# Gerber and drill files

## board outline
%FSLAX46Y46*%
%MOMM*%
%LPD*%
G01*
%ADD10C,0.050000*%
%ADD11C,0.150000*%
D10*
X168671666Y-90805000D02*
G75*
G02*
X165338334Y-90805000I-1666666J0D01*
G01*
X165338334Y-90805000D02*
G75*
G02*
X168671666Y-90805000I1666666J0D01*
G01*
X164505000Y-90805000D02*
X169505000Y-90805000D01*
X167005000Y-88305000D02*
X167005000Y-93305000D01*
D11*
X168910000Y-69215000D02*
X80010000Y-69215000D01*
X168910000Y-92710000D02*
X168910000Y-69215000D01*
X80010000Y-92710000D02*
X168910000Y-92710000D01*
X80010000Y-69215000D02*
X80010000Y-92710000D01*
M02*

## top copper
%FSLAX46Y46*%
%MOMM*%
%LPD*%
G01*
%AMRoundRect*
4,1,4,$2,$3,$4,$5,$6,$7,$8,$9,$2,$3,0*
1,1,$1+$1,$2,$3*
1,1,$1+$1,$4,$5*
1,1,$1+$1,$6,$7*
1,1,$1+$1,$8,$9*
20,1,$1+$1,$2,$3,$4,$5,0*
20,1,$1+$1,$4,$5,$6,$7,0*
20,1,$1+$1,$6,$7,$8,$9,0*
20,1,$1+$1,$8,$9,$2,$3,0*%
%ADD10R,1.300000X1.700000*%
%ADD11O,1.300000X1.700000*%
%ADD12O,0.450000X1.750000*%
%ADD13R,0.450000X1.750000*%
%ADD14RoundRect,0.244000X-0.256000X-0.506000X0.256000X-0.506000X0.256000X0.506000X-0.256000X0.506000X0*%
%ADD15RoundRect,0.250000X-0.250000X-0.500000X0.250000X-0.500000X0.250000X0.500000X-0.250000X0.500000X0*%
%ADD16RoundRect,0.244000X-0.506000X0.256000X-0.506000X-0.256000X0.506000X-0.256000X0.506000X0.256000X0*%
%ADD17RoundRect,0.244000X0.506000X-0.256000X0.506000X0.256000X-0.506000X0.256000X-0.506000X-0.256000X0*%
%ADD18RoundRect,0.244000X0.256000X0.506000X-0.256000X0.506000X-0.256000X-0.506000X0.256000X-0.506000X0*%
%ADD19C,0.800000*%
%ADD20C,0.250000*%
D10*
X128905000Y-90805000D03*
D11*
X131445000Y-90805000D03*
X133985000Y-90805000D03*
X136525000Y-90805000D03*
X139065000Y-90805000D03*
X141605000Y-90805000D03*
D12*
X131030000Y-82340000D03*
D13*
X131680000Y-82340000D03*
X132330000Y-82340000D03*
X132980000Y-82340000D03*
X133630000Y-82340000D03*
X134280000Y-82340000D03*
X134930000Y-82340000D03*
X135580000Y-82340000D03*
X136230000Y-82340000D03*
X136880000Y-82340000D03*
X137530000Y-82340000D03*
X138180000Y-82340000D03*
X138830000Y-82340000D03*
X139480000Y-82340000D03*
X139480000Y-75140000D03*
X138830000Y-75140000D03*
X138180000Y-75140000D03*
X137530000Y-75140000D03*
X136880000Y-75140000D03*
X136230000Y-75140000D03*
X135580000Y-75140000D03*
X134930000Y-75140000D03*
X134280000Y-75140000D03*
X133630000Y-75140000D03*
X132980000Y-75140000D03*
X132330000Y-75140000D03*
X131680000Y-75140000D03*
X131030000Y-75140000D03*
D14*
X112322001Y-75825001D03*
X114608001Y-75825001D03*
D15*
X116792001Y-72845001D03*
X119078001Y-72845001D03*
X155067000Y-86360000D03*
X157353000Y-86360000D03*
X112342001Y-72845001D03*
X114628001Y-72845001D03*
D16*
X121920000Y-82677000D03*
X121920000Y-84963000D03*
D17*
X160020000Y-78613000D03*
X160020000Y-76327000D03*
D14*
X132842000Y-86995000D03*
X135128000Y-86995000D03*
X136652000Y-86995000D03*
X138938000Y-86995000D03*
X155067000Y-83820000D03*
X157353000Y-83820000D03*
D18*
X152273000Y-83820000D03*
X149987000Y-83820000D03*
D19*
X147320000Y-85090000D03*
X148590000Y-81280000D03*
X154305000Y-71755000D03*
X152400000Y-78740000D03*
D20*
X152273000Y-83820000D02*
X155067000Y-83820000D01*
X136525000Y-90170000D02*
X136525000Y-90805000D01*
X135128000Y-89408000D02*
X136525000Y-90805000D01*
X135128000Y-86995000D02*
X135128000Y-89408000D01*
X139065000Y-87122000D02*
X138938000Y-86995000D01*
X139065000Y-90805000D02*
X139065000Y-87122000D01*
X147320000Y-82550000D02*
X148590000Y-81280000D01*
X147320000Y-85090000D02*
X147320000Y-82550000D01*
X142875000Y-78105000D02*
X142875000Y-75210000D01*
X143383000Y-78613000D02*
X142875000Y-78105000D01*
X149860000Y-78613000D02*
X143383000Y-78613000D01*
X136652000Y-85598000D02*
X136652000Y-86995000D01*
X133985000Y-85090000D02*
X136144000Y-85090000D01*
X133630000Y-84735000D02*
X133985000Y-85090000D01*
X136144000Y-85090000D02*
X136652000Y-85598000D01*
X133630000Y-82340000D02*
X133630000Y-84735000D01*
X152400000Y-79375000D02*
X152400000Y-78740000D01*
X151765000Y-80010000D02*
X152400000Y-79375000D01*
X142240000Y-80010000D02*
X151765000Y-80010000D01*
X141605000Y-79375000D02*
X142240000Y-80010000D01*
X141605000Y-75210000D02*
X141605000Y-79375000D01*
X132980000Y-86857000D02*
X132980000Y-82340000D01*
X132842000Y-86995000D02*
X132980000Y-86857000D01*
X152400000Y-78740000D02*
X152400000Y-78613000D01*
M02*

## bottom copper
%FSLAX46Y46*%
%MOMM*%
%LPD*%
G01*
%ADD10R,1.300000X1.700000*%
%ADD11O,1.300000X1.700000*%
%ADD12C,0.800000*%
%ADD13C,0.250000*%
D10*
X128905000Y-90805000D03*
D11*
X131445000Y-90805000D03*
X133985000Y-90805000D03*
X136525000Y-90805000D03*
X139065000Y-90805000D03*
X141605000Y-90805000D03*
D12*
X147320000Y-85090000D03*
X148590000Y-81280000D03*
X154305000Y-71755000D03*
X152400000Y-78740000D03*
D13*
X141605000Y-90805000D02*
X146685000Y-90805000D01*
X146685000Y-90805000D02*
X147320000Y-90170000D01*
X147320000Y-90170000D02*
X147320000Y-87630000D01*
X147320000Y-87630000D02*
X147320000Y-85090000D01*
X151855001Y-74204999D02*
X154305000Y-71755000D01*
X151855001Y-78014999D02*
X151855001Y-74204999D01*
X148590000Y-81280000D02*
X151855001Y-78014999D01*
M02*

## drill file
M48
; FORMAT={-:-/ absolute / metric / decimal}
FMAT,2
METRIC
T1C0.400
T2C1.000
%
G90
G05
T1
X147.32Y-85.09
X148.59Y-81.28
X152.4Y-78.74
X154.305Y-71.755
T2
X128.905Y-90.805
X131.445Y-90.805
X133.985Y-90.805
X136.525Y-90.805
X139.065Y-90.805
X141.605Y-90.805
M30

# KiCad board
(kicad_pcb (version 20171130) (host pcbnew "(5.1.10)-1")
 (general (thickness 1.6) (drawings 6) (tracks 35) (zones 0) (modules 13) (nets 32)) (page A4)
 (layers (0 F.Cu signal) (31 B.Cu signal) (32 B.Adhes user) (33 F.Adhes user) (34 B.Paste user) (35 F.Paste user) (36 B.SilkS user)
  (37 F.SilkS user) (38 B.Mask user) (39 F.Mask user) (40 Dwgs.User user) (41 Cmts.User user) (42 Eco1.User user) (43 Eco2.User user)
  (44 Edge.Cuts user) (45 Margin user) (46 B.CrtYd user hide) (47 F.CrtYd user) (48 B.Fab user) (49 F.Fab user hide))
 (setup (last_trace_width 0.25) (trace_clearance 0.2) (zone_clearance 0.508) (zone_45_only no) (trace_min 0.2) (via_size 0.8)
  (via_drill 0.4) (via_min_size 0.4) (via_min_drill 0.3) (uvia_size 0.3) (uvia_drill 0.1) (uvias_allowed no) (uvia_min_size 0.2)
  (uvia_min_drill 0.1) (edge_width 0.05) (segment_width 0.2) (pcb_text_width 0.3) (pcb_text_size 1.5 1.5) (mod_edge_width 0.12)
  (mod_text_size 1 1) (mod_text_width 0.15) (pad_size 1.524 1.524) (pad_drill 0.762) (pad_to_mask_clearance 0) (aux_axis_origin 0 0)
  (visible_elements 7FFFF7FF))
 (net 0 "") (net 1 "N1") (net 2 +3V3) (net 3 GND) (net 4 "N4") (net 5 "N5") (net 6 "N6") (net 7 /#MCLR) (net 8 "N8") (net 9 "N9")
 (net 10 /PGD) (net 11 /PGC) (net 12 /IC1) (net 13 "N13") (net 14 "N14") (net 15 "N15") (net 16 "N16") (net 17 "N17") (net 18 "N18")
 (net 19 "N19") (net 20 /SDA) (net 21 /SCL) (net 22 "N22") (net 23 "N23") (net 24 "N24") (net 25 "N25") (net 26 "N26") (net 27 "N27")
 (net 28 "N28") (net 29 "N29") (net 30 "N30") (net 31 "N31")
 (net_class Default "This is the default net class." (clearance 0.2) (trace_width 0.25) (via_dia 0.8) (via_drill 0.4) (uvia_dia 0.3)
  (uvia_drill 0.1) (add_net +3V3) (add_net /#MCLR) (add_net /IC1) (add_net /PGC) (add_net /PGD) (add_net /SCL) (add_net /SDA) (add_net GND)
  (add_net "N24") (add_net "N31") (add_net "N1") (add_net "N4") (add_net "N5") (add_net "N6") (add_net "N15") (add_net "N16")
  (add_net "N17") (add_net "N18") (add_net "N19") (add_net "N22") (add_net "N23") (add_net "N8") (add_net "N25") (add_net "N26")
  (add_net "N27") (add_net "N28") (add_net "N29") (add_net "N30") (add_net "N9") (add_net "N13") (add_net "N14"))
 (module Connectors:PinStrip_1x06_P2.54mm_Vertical (layer F.Cu) (at 128.905 90.805 90)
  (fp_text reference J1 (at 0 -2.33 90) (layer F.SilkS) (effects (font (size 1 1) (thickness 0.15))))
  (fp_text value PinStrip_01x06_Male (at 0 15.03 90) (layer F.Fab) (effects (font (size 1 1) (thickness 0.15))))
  (pad 1 thru_hole rect (at 0 0 90) (size 1.7 1.3) (drill 1) (layers *.Cu *.Mask) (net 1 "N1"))
  (pad 2 thru_hole oval (at 0 2.54 90) (size 1.7 1.3) (drill 1) (layers *.Cu *.Mask) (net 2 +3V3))
  (pad 3 thru_hole oval (at 0 5.08 90) (size 1.7 1.3) (drill 1) (layers *.Cu *.Mask) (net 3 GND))
  (pad 4 thru_hole oval (at 0 7.62 90) (size 1.7 1.3) (drill 1) (layers *.Cu *.Mask) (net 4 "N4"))
  (pad 5 thru_hole oval (at 0 10.16 90) (size 1.7 1.3) (drill 1) (layers *.Cu *.Mask) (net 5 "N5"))
  (pad 6 thru_hole oval (at 0 12.7 90) (size 1.7 1.3) (drill 1) (layers *.Cu *.Mask) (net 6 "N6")))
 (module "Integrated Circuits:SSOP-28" (layer F.Cu) (at 135.255 78.74 90)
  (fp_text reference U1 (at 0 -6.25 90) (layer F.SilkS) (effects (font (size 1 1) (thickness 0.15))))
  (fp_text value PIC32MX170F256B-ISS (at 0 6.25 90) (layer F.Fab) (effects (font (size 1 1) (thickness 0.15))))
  (pad 1 smd oval (at -3.6 -4.225 90) (size 1.75 0.45) (layers F.Cu F.Paste F.Mask) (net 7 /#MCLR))
  (pad 2 smd rect (at -3.6 -3.575 90) (size 1.75 0.45) (layers F.Cu F.Paste F.Mask) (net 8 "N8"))
  (pad 3 smd rect (at -3.6 -2.925 90) (size 1.75 0.45) (layers F.Cu F.Paste F.Mask) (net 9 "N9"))
  (pad 4 smd rect (at -3.6 -2.275 90) (size 1.75 0.45) (layers F.Cu F.Paste F.Mask) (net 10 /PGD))
  (pad 5 smd rect (at -3.6 -1.625 90) (size 1.75 0.45) (layers F.Cu F.Paste F.Mask) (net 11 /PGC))
  (pad 6 smd rect (at -3.6 -0.975 90) (size 1.75 0.45) (layers F.Cu F.Paste F.Mask) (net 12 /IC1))
  (pad 7 smd rect (at -3.6 -0.325 90) (size 1.75 0.45) (layers F.Cu F.Paste F.Mask) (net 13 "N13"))
  (pad 8 smd rect (at -3.6 0.325 90) (size 1.75 0.45) (layers F.Cu F.Paste F.Mask) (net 3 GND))
  (pad 9 smd rect (at -3.6 0.975 90) (size 1.75 0.45) (layers F.Cu F.Paste F.Mask) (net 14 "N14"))
  (pad 10 smd rect (at -3.6 1.625 90) (size 1.75 0.45) (layers F.Cu F.Paste F.Mask) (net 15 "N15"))
  (pad 11 smd rect (at -3.6 2.275 90) (size 1.75 0.45) (layers F.Cu F.Paste F.Mask) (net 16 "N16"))
  (pad 12 smd rect (at -3.6 2.925 90) (size 1.75 0.45) (layers F.Cu F.Paste F.Mask) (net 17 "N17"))
  (pad 13 smd rect (at -3.6 3.575 90) (size 1.75 0.45) (layers F.Cu F.Paste F.Mask) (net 2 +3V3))
  (pad 14 smd rect (at -3.6 4.225 90) (size 1.75 0.45) (layers F.Cu F.Paste F.Mask) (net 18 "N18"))
  (pad 15 smd rect (at 3.6 4.225 90) (size 1.75 0.45) (layers F.Cu F.Paste F.Mask) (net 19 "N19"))
  (pad 16 smd rect (at 3.6 3.575 90) (size 1.75 0.45) (layers F.Cu F.Paste F.Mask) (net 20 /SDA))
  (pad 17 smd rect (at 3.6 2.925 90) (size 1.75 0.45) (layers F.Cu F.Paste F.Mask) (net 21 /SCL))
  (pad 18 smd rect (at 3.6 2.275 90) (size 1.75 0.45) (layers F.Cu F.Paste F.Mask) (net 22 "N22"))
  (pad 19 smd rect (at 3.6 1.625 90) (size 1.75 0.45) (layers F.Cu F.Paste F.Mask) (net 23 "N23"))
  (pad 20 smd rect (at 3.6 0.975 90) (size 1.75 0.45) (layers F.Cu F.Paste F.Mask) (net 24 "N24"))
  (pad 21 smd rect (at 3.6 0.325 90) (size 1.75 0.45) (layers F.Cu F.Paste F.Mask) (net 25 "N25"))
  (pad 22 smd rect (at 3.6 -0.325 90) (size 1.75 0.45) (layers F.Cu F.Paste F.Mask) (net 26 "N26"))
  (pad 23 smd rect (at 3.6 -0.975 90) (size 1.75 0.45) (layers F.Cu F.Paste F.Mask) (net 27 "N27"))
  (pad 24 smd rect (at 3.6 -1.625 90) (size 1.75 0.45) (layers F.Cu F.Paste F.Mask) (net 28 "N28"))
  (pad 25 smd rect (at 3.6 -2.275 90) (size 1.75 0.45) (layers F.Cu F.Paste F.Mask) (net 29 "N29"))
  (pad 26 smd rect (at 3.6 -2.925 90) (size 1.75 0.45) (layers F.Cu F.Paste F.Mask) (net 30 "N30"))
  (pad 27 smd rect (at 3.6 -3.575 90) (size 1.75 0.45) (layers F.Cu F.Paste F.Mask) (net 3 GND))
  (pad 28 smd rect (at 3.6 -4.225 90) (size 1.75 0.45) (layers F.Cu F.Paste F.Mask) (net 2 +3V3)))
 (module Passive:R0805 (layer F.Cu) (at 113.465001 75.825001)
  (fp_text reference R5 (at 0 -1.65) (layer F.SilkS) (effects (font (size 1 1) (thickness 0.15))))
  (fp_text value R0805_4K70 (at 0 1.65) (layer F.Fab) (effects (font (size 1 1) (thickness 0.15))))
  (pad 1 smd roundrect (at -1.143 0) (size 1 1.5) (layers F.Cu F.Paste F.Mask) (roundrect_rratio 0.244) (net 2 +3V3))
  (pad 2 smd roundrect (at 1.143 0) (size 1 1.5) (layers F.Cu F.Paste F.Mask) (roundrect_rratio 0.244) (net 7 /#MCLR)))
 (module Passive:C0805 (layer F.Cu) (at 117.935001 72.845001)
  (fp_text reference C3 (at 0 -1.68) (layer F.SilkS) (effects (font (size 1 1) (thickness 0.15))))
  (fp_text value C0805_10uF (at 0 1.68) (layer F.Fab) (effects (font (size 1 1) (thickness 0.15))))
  (pad 1 smd roundrect (at -1.143 0) (size 1 1.5) (layers F.Cu F.Paste F.Mask) (roundrect_rratio 0.25) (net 24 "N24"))
  (pad 2 smd roundrect (at 1.143 0) (size 1 1.5) (layers F.Cu F.Paste F.Mask) (roundrect_rratio 0.25) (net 3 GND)))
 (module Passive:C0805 (layer F.Cu) (at 156.21 86.36)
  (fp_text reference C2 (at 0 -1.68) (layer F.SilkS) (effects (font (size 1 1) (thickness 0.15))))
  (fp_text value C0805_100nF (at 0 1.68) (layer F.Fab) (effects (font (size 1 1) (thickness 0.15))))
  (pad 1 smd roundrect (at -1.143 0) (size 1 1.5) (layers F.Cu F.Paste F.Mask) (roundrect_rratio 0.25) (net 2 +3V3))
  (pad 2 smd roundrect (at 1.143 0) (size 1 1.5) (layers F.Cu F.Paste F.Mask) (roundrect_rratio 0.25) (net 3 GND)))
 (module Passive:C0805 (layer F.Cu) (at 113.485001 72.845001)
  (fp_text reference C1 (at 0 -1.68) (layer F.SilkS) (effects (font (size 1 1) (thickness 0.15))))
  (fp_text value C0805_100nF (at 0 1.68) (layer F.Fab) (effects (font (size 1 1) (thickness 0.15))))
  (pad 1 smd roundrect (at -1.143 0) (size 1 1.5) (layers F.Cu F.Paste F.Mask) (roundrect_rratio 0.25) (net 2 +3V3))
  (pad 2 smd roundrect (at 1.143 0) (size 1 1.5) (layers F.Cu F.Paste F.Mask) (roundrect_rratio 0.25) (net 3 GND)))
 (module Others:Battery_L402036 (layer F.Cu) (at 143.51 70.485 180)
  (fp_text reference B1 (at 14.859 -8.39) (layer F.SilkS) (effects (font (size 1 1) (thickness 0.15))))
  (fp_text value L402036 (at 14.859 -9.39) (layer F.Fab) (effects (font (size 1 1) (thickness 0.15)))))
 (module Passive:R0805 (layer F.Cu) (at 121.92 83.82 270)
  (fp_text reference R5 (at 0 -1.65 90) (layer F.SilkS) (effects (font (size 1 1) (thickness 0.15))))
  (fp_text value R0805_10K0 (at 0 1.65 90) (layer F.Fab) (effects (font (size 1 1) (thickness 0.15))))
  (pad 1 smd roundrect (at -1.143 0 270) (size 1 1.5) (layers F.Cu F.Paste F.Mask) (roundrect_rratio 0.244) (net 2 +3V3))
  (pad 2 smd roundrect (at 1.143 0 270) (size 1 1.5) (layers F.Cu F.Paste F.Mask) (roundrect_rratio 0.244) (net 7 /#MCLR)))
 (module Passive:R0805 (layer F.Cu) (at 160.02 77.47 90)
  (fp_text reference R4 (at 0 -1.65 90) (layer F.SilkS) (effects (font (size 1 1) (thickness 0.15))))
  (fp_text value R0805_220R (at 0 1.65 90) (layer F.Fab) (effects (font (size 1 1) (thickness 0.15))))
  (pad 1 smd roundrect (at -1.143 0 90) (size 1 1.5) (layers F.Cu F.Paste F.Mask) (roundrect_rratio 0.244) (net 7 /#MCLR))
  (pad 2 smd roundrect (at 1.143 0 90) (size 1 1.5) (layers F.Cu F.Paste F.Mask) (roundrect_rratio 0.244) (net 1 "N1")))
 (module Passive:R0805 (layer F.Cu) (at 133.985 86.995)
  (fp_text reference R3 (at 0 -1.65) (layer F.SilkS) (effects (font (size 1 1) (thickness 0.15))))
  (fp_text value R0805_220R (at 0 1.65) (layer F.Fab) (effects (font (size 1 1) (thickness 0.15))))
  (pad 1 smd roundrect (at -1.143 0) (size 1 1.5) (layers F.Cu F.Paste F.Mask) (roundrect_rratio 0.244) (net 10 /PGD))
  (pad 2 smd roundrect (at 1.143 0) (size 1 1.5) (layers F.Cu F.Paste F.Mask) (roundrect_rratio 0.244) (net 4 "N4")))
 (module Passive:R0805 (layer F.Cu) (at 137.795 86.995)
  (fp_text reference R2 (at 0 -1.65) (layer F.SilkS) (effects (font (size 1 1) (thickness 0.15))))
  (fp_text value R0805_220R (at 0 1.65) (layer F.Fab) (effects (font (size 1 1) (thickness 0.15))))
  (pad 1 smd roundrect (at -1.143 0) (size 1 1.5) (layers F.Cu F.Paste F.Mask) (roundrect_rratio 0.244) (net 11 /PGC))
  (pad 2 smd roundrect (at 1.143 0) (size 1 1.5) (layers F.Cu F.Paste F.Mask) (roundrect_rratio 0.244) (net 5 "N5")))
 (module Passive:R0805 (layer F.Cu) (at 156.21 83.82)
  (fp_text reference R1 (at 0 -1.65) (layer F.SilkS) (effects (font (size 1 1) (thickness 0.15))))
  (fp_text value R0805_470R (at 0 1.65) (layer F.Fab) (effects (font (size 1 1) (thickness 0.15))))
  (pad 1 smd roundrect (at -1.143 0) (size 1 1.5) (layers F.Cu F.Paste F.Mask) (roundrect_rratio 0.244) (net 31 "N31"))
  (pad 2 smd roundrect (at 1.143 0) (size 1 1.5) (layers F.Cu F.Paste F.Mask) (roundrect_rratio 0.244) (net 3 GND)))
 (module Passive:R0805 (layer F.Cu) (at 151.13 83.82 180)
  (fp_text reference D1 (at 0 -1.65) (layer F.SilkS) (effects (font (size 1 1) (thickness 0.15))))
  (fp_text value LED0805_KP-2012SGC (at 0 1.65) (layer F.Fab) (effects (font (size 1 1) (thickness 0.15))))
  (pad 1 smd roundrect (at -1.143 0 180) (size 1 1.5) (layers F.Cu F.Paste F.Mask) (roundrect_rratio 0.244) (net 31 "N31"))
  (pad 2 smd roundrect (at 1.143 0 180) (size 1 1.5) (layers F.Cu F.Paste F.Mask) (roundrect_rratio 0.244) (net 2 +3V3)))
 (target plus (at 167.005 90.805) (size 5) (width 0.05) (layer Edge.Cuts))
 (gr_line (start 168.91 69.215) (end 80.01 69.215) (layer Edge.Cuts) (width 0.15))
 (gr_line (start 168.91 92.71) (end 168.91 69.215) (layer Edge.Cuts) (width 0.15))
 (gr_line (start 80.01 92.71) (end 168.91 92.71) (layer Edge.Cuts) (width 0.15))
 (gr_line (start 80.01 69.215) (end 80.01 92.71) (layer Edge.Cuts) (width 0.15))
 (segment (start 152.273 83.82) (end 155.067 83.82) (width 0.25) (layer F.Cu) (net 31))
 (segment (start 136.525 90.17) (end 136.525 90.805) (width 0.25) (layer F.Cu) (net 4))
 (segment (start 135.128 89.408) (end 136.525 90.805) (width 0.25) (layer F.Cu) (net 4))
 (segment (start 135.128 86.995) (end 135.128 89.408) (width 0.25) (layer F.Cu) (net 4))
 (segment (start 139.065 87.122) (end 138.938 86.995) (width 0.25) (layer F.Cu) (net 5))
 (segment (start 139.065 90.805) (end 139.065 87.122) (width 0.25) (layer F.Cu) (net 5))
 (segment (start 141.605 90.805) (end 146.685 90.805) (width 0.25) (layer B.Cu) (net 6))
 (segment (start 146.685 90.805) (end 147.32 90.17) (width 0.25) (layer B.Cu) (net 6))
 (segment (start 147.32 90.17) (end 147.32 87.63) (width 0.25) (layer B.Cu) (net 6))
 (via (at 147.32 85.09) (size 0.8) (drill 0.4) (layers F.Cu B.Cu) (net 6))
 (segment (start 147.32 87.63) (end 147.32 85.09) (width 0.25) (layer B.Cu) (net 6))
 (via (at 148.59 81.28) (size 0.8) (drill 0.4) (layers F.Cu B.Cu) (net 6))
 (segment (start 147.32 82.55) (end 148.59 81.28) (width 0.25) (layer F.Cu) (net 6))
 (segment (start 147.32 85.09) (end 147.32 82.55) (width 0.25) (layer F.Cu) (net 6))
 (via (at 154.305 71.755) (size 0.8) (drill 0.4) (layers F.Cu B.Cu) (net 6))
 (segment (start 151.855001 74.204999) (end 154.305 71.755) (width 0.25) (layer B.Cu) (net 6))
 (segment (start 151.855001 78.014999) (end 151.855001 74.204999) (width 0.25) (layer B.Cu) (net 6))
 (segment (start 148.59 81.28) (end 151.855001 78.014999) (width 0.25) (layer B.Cu) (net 6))
 (segment (start 142.875 78.105) (end 142.875 75.21) (width 0.25) (layer F.Cu) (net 11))
 (segment (start 143.383 78.613) (end 142.875 78.105) (width 0.25) (layer F.Cu) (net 11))
 (segment (start 149.86 78.613) (end 143.383 78.613) (width 0.25) (layer F.Cu) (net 11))
 (segment (start 136.652 85.598) (end 136.652 86.995) (width 0.25) (layer F.Cu) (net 11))
 (segment (start 133.985 85.09) (end 136.144 85.09) (width 0.25) (layer F.Cu) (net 11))
 (segment (start 133.63 84.735) (end 133.985 85.09) (width 0.25) (layer F.Cu) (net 11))
 (segment (start 136.144 85.09) (end 136.652 85.598) (width 0.25) (layer F.Cu) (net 11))
 (segment (start 133.63 82.34) (end 133.63 84.735) (width 0.25) (layer F.Cu) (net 11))
 (segment (start 152.4 79.375) (end 152.4 78.74) (width 0.25) (layer F.Cu) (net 10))
 (segment (start 151.765 80.01) (end 152.4 79.375) (width 0.25) (layer F.Cu) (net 10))
 (segment (start 142.24 80.01) (end 151.765 80.01) (width 0.25) (layer F.Cu) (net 10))
 (segment (start 141.605 79.375) (end 142.24 80.01) (width 0.25) (layer F.Cu) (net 10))
 (segment (start 141.605 75.21) (end 141.605 79.375) (width 0.25) (layer F.Cu) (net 10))
 (segment (start 132.98 86.857) (end 132.98 82.34) (width 0.25) (layer F.Cu) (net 10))
 (segment (start 132.842 86.995) (end 132.98 86.857) (width 0.25) (layer F.Cu) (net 10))
 (segment (start 152.4 78.74) (end 152.4 78.613) (width 0.25) (layer F.Cu) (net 10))
 (via (at 152.4 78.74) (size 0.8) (drill 0.4) (layers F.Cu B.Cu) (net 10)))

